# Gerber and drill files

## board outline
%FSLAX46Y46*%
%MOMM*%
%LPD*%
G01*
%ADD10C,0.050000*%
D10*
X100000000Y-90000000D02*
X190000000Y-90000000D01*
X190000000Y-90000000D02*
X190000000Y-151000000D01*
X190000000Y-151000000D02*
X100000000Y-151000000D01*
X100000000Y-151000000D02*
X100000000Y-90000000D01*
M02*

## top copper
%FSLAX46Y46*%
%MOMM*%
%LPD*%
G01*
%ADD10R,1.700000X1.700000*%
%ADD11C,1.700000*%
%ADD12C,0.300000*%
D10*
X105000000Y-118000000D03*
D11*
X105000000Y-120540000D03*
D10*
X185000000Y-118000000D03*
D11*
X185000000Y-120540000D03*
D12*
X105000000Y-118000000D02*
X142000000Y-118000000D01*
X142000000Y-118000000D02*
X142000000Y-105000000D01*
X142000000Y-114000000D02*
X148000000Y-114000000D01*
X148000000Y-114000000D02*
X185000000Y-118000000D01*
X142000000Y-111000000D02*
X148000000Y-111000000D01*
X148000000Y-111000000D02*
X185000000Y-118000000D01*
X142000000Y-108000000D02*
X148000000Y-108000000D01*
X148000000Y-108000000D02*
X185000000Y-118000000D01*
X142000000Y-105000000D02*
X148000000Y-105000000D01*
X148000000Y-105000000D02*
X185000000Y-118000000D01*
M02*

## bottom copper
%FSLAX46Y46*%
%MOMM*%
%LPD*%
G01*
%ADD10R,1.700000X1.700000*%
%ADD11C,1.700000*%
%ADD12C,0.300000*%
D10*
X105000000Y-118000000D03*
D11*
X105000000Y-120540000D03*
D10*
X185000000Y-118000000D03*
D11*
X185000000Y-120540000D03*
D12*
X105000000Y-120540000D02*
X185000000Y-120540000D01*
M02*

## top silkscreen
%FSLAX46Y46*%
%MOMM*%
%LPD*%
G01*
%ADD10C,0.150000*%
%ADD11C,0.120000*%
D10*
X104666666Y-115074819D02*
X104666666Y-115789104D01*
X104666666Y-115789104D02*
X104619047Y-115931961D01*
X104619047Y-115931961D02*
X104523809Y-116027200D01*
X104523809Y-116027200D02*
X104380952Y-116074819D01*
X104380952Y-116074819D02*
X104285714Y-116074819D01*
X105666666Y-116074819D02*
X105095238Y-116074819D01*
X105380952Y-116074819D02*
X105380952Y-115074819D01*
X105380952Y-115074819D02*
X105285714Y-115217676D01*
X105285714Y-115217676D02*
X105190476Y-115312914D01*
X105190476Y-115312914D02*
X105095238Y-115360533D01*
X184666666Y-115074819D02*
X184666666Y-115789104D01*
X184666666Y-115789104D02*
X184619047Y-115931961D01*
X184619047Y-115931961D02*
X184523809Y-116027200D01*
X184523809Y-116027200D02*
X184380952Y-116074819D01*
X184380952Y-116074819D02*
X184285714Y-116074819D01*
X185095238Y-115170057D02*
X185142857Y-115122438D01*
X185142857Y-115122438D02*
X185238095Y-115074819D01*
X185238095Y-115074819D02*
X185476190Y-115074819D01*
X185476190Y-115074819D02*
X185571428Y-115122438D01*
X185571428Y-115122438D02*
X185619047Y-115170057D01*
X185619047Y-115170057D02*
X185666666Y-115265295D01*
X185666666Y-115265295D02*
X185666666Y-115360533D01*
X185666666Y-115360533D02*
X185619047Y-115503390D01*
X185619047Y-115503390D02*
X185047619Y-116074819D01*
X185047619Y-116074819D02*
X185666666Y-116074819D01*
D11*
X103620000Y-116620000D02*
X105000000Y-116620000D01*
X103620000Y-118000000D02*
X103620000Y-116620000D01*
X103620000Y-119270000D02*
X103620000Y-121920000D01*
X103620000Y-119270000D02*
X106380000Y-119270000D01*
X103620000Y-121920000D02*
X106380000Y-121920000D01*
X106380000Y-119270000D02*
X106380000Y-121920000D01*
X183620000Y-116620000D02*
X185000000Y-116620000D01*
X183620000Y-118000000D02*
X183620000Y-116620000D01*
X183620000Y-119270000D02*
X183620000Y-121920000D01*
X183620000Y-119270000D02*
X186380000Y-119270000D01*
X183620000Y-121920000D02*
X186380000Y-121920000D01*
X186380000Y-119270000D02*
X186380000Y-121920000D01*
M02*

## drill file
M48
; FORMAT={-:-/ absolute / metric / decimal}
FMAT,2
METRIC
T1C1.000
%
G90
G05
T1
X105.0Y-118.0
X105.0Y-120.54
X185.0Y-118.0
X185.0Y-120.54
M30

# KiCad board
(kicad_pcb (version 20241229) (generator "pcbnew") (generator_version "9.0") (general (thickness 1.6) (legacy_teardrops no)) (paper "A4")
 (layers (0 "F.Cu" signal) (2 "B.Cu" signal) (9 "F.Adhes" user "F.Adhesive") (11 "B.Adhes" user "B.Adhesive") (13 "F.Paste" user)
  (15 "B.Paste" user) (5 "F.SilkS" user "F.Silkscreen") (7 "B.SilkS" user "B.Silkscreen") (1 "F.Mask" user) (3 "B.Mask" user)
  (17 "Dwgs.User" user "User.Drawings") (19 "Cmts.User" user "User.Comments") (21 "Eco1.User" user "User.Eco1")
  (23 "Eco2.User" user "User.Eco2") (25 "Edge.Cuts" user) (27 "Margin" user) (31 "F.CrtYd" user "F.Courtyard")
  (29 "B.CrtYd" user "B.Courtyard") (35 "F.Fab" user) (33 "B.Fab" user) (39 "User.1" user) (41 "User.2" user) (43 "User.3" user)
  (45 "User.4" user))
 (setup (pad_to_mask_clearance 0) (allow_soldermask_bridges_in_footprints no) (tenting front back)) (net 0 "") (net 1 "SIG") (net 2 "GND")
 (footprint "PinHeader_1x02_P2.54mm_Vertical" (layer "F.Cu") (at 105 118)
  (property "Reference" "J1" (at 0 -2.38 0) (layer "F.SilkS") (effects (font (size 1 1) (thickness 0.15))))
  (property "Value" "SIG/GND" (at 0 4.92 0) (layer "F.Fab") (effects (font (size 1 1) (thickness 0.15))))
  (fp_line (start -1.38 -1.38) (end 0 -1.38) (stroke (width 0.12) (type solid)) (layer "F.SilkS"))
  (fp_line (start -1.38 0) (end -1.38 -1.38) (stroke (width 0.12) (type solid)) (layer "F.SilkS"))
  (fp_line (start -1.38 1.27) (end -1.38 3.92) (stroke (width 0.12) (type solid)) (layer "F.SilkS"))
  (fp_line (start -1.38 1.27) (end 1.38 1.27) (stroke (width 0.12) (type solid)) (layer "F.SilkS"))
  (fp_line (start -1.38 3.92) (end 1.38 3.92) (stroke (width 0.12) (type solid)) (layer "F.SilkS"))
  (fp_line (start 1.38 1.27) (end 1.38 3.92) (stroke (width 0.12) (type solid)) (layer "F.SilkS"))
  (pad "1" thru_hole rect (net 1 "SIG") (at 0 0) (size 1.7 1.7) (drill 1) (layers "*.Cu" "*.Mask") (remove_unused_layers no))
  (pad "2" thru_hole circle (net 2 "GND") (at 0 2.54) (size 1.7 1.7) (drill 1) (layers "*.Cu" "*.Mask") (remove_unused_layers no)))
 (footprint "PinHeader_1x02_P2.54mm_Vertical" (layer "F.Cu") (at 185 118)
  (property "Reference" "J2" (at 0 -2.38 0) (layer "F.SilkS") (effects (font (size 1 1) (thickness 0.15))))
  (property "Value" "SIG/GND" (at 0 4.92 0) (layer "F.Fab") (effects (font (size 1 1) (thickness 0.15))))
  (fp_line (start -1.38 -1.38) (end 0 -1.38) (stroke (width 0.12) (type solid)) (layer "F.SilkS"))
  (fp_line (start -1.38 0) (end -1.38 -1.38) (stroke (width 0.12) (type solid)) (layer "F.SilkS"))
  (fp_line (start -1.38 1.27) (end -1.38 3.92) (stroke (width 0.12) (type solid)) (layer "F.SilkS"))
  (fp_line (start -1.38 1.27) (end 1.38 1.27) (stroke (width 0.12) (type solid)) (layer "F.SilkS"))
  (fp_line (start -1.38 3.92) (end 1.38 3.92) (stroke (width 0.12) (type solid)) (layer "F.SilkS"))
  (fp_line (start 1.38 1.27) (end 1.38 3.92) (stroke (width 0.12) (type solid)) (layer "F.SilkS"))
  (pad "1" thru_hole rect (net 1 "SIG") (at 0 0) (size 1.7 1.7) (drill 1) (layers "*.Cu" "*.Mask") (remove_unused_layers no))
  (pad "2" thru_hole circle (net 2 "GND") (at 0 2.54) (size 1.7 1.7) (drill 1) (layers "*.Cu" "*.Mask") (remove_unused_layers no)))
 (gr_line (start 100 90) (end 190 90) (stroke (width 0.05) (type solid)) (layer "Edge.Cuts"))
 (gr_line (start 190 90) (end 190 151) (stroke (width 0.05) (type solid)) (layer "Edge.Cuts"))
 (gr_line (start 190 151) (end 100 151) (stroke (width 0.05) (type solid)) (layer "Edge.Cuts"))
 (gr_line (start 100 151) (end 100 90) (stroke (width 0.05) (type solid)) (layer "Edge.Cuts"))
 (segment (start 105 120.54) (end 185 120.54) (width 0.3) (layer "B.Cu") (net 2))
 (segment (start 105 118) (end 142 118) (width 0.3) (layer "F.Cu") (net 1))
 (segment (start 142 118) (end 142 105) (width 0.3) (layer "F.Cu") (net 1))
 (segment (start 142 114) (end 148 114) (width 0.3) (layer "F.Cu") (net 1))
 (segment (start 148 114) (end 185 118) (width 0.3) (layer "F.Cu") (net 1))
 (segment (start 142 111) (end 148 111) (width 0.3) (layer "F.Cu") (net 1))
 (segment (start 148 111) (end 185 118) (width 0.3) (layer "F.Cu") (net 1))
 (segment (start 142 108) (end 148 108) (width 0.3) (layer "F.Cu") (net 1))
 (segment (start 148 108) (end 185 118) (width 0.3) (layer "F.Cu") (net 1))
 (segment (start 142 105) (end 148 105) (width 0.3) (layer "F.Cu") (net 1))
 (segment (start 148 105) (end 185 118) (width 0.3) (layer "F.Cu") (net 1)))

